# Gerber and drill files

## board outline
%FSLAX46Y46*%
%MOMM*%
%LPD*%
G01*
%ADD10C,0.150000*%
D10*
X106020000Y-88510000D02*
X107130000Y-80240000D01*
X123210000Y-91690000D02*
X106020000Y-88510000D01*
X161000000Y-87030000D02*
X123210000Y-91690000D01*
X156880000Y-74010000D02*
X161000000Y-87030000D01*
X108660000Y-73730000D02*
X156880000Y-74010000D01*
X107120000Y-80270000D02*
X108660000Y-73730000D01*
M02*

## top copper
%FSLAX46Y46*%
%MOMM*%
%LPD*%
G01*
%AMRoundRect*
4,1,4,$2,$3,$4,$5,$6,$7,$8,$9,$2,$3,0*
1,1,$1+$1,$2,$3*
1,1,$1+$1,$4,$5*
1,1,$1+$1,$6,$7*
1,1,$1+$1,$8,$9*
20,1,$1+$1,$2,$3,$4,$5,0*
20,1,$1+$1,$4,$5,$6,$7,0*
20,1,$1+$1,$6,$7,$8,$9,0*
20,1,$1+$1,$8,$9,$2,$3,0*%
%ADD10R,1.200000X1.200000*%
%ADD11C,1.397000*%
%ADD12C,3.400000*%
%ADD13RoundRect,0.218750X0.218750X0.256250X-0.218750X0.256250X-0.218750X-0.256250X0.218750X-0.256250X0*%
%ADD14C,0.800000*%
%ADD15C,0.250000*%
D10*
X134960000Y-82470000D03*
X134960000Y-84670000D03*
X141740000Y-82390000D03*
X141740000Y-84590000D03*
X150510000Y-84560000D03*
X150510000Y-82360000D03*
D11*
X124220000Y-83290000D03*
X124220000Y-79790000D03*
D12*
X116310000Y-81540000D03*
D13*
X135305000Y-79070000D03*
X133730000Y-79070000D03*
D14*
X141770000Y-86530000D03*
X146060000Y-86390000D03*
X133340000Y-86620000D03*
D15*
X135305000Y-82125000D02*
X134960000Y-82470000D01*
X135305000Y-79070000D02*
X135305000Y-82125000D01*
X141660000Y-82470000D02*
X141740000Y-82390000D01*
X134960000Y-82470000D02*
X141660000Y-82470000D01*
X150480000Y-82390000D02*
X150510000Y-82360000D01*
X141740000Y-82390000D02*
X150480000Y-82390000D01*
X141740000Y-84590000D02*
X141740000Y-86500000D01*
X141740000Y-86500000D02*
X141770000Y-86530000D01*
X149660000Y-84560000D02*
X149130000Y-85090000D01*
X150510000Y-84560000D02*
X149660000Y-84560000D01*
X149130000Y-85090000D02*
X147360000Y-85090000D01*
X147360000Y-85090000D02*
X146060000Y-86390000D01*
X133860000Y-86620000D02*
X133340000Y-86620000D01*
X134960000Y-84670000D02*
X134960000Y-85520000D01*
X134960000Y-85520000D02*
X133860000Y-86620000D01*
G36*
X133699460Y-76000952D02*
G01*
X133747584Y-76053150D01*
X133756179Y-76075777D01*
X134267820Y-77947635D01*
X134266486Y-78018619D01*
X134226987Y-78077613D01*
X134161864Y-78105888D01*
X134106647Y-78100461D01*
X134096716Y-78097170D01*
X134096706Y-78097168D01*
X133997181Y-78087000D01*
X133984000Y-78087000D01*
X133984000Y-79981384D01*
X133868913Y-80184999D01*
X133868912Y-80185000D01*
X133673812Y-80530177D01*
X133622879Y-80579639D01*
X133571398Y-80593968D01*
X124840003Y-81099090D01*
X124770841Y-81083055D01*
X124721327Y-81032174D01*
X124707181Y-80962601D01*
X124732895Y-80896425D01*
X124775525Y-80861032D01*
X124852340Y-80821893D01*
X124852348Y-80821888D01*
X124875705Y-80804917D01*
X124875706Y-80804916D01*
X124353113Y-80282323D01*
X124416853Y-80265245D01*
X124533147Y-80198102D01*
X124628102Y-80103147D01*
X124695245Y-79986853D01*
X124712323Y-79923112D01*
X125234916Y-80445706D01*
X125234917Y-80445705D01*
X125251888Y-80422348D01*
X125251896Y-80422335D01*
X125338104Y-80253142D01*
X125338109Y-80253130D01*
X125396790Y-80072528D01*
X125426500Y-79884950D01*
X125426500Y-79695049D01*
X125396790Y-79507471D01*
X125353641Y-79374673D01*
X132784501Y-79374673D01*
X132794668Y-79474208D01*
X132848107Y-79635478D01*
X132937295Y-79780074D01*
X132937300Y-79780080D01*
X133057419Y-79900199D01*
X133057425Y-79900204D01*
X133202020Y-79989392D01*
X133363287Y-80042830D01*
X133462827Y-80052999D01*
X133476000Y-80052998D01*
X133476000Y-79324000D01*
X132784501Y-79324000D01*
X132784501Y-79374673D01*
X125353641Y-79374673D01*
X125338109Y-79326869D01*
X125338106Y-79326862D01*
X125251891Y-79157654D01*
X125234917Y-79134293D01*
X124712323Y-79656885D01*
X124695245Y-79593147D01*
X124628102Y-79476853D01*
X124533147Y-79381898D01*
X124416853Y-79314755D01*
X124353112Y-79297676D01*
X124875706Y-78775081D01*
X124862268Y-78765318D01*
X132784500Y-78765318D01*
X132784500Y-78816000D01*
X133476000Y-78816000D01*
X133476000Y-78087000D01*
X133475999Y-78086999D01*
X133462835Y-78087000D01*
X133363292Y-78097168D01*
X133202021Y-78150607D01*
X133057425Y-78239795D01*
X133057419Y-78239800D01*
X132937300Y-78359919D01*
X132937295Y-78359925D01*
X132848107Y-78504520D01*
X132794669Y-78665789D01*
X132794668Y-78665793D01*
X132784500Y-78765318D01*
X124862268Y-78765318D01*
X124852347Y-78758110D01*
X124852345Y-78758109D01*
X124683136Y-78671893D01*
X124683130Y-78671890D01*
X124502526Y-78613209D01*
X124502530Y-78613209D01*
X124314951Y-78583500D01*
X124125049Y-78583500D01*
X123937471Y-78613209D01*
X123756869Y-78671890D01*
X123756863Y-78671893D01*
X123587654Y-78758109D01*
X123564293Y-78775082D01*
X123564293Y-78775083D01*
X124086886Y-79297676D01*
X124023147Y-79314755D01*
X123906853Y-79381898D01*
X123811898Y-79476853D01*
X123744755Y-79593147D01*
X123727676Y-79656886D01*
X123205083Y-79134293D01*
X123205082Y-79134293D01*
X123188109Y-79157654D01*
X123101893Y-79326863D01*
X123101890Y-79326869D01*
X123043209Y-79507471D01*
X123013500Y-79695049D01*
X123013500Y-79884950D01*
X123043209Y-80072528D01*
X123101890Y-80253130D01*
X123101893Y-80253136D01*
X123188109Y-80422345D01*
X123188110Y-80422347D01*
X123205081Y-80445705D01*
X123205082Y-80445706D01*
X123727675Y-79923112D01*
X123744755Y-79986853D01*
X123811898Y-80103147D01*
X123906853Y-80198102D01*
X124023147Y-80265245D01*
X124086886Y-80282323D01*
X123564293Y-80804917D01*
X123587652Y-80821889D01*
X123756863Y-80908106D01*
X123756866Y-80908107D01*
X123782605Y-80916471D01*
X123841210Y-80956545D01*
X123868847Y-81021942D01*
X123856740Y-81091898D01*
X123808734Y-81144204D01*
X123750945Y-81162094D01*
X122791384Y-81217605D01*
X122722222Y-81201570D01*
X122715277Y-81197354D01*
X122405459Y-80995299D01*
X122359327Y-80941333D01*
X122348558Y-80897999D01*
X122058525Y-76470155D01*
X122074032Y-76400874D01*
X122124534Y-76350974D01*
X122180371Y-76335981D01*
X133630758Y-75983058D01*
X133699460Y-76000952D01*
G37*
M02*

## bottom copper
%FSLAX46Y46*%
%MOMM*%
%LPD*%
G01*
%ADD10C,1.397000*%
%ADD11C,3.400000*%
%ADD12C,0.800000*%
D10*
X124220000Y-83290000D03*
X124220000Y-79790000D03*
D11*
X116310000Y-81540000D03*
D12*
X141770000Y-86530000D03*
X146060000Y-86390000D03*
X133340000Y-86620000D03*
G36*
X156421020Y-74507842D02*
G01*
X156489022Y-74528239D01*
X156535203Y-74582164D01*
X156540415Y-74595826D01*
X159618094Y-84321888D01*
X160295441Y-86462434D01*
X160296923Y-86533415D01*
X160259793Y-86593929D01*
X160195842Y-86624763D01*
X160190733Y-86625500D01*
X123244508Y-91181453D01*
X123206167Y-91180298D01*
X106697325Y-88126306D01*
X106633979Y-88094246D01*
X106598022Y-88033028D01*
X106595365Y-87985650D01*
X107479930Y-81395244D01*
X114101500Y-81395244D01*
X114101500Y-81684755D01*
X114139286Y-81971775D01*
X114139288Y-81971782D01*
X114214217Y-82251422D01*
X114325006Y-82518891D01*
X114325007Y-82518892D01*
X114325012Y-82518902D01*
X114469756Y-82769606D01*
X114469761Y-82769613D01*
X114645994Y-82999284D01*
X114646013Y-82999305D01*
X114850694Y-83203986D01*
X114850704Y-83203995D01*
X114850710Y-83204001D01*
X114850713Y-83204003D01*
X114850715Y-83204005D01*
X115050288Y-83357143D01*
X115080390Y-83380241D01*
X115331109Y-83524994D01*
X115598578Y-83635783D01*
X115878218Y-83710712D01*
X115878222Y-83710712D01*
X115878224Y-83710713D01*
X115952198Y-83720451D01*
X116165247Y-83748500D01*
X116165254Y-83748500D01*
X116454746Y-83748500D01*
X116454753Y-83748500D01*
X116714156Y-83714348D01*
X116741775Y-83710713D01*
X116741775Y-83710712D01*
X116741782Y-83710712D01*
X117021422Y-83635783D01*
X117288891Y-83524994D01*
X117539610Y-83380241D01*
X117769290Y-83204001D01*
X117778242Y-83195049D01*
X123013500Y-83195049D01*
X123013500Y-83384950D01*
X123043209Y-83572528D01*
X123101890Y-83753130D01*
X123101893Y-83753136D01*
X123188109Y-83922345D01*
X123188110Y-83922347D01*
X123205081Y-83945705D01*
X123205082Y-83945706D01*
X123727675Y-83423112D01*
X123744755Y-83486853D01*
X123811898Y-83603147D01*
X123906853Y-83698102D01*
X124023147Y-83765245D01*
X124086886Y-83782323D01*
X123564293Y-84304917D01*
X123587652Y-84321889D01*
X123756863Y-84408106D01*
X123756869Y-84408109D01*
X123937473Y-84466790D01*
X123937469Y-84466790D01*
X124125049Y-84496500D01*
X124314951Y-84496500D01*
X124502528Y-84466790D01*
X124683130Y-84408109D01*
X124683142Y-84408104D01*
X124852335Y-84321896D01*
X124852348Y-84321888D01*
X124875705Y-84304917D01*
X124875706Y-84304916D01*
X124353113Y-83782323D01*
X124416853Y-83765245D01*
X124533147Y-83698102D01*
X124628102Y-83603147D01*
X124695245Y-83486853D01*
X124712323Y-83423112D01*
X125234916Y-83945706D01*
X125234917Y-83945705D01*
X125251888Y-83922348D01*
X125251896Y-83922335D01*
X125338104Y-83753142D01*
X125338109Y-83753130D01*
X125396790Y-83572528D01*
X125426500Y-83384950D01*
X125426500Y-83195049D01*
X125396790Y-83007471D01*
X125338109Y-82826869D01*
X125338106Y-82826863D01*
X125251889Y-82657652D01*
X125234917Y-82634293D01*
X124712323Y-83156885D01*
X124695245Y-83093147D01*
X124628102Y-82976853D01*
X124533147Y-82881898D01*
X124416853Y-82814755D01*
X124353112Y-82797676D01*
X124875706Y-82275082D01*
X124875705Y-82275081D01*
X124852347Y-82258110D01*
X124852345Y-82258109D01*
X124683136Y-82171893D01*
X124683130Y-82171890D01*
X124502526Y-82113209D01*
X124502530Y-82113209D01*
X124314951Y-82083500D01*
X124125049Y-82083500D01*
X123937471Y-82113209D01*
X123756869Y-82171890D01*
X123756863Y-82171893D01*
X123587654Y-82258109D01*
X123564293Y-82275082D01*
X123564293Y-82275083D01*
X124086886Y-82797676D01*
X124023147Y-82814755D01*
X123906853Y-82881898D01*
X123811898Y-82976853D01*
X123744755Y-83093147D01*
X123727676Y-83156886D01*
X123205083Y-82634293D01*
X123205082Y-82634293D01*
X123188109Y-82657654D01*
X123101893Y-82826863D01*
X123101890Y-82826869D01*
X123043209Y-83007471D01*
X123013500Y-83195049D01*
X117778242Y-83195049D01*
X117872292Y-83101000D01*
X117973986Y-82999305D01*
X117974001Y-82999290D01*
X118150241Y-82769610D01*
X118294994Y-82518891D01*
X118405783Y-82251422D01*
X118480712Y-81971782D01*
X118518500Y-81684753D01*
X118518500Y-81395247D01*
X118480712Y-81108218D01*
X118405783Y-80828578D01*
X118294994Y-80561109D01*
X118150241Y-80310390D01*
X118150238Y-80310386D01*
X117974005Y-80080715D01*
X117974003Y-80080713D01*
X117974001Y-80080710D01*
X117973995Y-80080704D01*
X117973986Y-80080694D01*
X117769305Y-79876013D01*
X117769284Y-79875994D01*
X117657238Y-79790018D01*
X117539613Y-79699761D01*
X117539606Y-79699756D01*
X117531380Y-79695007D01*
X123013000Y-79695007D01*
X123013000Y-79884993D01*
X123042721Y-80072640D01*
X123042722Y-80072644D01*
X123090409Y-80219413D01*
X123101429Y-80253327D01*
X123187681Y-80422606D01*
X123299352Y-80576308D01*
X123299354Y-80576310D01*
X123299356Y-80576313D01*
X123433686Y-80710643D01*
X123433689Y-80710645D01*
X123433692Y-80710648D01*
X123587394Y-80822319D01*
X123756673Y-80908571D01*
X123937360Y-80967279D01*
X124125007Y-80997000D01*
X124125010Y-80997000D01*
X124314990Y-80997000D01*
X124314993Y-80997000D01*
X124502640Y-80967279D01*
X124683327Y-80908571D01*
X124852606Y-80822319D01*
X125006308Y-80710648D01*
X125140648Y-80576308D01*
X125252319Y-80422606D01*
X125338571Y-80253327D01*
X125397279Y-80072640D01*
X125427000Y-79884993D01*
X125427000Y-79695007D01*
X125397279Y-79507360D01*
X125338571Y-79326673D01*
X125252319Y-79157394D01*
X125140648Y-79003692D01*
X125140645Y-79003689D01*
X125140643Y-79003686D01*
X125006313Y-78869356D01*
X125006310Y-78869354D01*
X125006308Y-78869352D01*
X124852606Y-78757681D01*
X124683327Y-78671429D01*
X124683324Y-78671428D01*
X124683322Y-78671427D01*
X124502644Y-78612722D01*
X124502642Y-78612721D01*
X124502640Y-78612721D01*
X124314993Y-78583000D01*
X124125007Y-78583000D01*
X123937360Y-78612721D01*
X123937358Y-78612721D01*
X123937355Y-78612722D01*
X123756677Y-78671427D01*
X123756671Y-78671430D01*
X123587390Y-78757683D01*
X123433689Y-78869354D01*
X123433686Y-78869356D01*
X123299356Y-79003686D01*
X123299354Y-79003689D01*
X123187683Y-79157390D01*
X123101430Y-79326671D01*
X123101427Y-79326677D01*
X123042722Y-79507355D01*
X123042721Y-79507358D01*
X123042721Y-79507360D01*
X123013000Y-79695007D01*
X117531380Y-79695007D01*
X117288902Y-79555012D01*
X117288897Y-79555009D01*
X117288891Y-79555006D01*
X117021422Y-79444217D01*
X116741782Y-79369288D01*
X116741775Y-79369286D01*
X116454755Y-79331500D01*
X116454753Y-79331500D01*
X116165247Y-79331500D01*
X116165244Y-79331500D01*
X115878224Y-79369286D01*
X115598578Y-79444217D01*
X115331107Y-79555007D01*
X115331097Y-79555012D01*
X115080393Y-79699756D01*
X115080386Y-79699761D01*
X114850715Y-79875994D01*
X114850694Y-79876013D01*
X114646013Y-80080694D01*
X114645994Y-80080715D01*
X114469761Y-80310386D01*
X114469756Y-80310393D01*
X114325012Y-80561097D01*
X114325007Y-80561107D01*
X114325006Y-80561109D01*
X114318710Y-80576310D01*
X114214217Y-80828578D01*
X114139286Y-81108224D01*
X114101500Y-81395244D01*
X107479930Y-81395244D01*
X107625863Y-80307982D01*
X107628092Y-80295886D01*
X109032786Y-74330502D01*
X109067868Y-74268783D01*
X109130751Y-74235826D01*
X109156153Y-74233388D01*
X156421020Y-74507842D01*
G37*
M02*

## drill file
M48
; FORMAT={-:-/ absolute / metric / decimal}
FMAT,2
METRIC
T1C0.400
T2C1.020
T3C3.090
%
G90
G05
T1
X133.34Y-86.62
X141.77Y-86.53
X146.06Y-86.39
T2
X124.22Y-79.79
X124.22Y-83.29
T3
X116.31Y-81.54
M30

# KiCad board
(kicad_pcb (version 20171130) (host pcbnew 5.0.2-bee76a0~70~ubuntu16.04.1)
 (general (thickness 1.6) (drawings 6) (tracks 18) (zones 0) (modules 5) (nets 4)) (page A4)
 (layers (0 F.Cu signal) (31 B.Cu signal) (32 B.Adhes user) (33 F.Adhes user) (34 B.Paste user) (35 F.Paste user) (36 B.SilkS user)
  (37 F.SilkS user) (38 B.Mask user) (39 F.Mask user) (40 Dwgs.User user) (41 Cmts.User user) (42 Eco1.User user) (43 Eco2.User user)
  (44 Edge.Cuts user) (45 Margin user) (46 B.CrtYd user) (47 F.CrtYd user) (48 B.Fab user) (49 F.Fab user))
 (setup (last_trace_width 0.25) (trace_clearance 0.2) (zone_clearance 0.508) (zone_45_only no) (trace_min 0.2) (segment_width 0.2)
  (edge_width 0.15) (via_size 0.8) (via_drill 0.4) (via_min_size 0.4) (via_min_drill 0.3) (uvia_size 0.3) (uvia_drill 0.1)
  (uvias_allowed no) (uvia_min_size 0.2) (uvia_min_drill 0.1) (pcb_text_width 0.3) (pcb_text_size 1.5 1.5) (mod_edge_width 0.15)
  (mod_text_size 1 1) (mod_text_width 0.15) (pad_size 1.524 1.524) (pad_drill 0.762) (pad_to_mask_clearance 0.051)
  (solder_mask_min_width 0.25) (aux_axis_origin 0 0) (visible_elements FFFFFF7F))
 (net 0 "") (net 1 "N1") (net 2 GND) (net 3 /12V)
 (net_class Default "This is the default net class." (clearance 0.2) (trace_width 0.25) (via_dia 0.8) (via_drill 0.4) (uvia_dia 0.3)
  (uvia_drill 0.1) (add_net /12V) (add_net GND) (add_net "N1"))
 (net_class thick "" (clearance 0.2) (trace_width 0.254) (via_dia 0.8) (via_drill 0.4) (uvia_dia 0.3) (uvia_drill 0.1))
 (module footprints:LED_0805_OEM (layer F.Cu) (at 134.96 83.57 90)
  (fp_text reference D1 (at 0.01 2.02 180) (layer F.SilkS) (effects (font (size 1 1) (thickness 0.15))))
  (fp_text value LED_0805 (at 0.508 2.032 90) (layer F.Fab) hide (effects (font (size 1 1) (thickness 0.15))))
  (pad 2 smd rect (at 1.1 0 270) (size 1.2 1.2) (layers F.Cu F.Paste F.Mask) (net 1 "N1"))
  (pad 1 smd rect (at -1.1 0 270) (size 1.2 1.2) (layers F.Cu F.Paste F.Mask) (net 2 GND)))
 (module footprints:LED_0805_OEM (layer F.Cu) (at 141.74 83.49 90)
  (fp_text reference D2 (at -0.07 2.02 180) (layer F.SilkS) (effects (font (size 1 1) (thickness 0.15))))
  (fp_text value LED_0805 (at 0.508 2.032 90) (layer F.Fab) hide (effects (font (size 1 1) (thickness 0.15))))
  (pad 2 smd rect (at 1.1 0 270) (size 1.2 1.2) (layers F.Cu F.Paste F.Mask) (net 1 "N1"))
  (pad 1 smd rect (at -1.1 0 270) (size 1.2 1.2) (layers F.Cu F.Paste F.Mask) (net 2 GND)))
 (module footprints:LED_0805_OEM (layer F.Cu) (at 150.51 83.46 90)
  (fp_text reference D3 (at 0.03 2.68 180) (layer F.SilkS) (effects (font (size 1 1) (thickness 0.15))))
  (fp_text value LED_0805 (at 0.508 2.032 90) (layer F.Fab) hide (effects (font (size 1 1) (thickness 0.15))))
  (pad 1 smd rect (at -1.1 0 270) (size 1.2 1.2) (layers F.Cu F.Paste F.Mask) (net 2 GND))
  (pad 2 smd rect (at 1.1 0 270) (size 1.2 1.2) (layers F.Cu F.Paste F.Mask) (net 1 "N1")))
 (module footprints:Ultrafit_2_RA (layer F.Cu) (at 124.22 83.29 180)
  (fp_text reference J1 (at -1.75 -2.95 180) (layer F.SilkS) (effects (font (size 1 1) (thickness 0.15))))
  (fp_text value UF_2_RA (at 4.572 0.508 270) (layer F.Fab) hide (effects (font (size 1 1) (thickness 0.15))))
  (pad 2 thru_hole circle (at 0 0 180) (size 1.397 1.397) (drill 1.02) (layers *.Cu *.Mask) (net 2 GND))
  (pad 1 thru_hole circle (at 0 3.5 180) (size 1.397 1.397) (drill 1.02) (layers *.Cu *.Mask) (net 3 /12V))
  (pad "" thru_hole circle (at 7.91 1.75 180) (size 3.4 3.4) (drill 3.09) (layers *.Cu *.Mask)))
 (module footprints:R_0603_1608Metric (layer F.Cu) (at 134.5175 79.07 180)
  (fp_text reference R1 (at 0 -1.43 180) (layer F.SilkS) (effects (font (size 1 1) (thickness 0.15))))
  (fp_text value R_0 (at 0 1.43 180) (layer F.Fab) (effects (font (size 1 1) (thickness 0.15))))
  (pad 1 smd roundrect (at -0.7875 0 180) (size 0.875 0.95) (layers F.Cu F.Paste F.Mask) (roundrect_rratio 0.25) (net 1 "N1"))
  (pad 2 smd roundrect (at 0.7875 0 180) (size 0.875 0.95) (layers F.Cu F.Paste F.Mask) (roundrect_rratio 0.25) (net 3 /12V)))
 (gr_line (start 106.02 88.51) (end 107.13 80.24) (layer Edge.Cuts) (width 0.15))
 (gr_line (start 123.21 91.69) (end 106.02 88.51) (layer Edge.Cuts) (width 0.15))
 (gr_line (start 161 87.03) (end 123.21 91.69) (layer Edge.Cuts) (width 0.15))
 (gr_line (start 156.88 74.01) (end 161 87.03) (layer Edge.Cuts) (width 0.15))
 (gr_line (start 108.66 73.73) (end 156.88 74.01) (layer Edge.Cuts) (width 0.15))
 (gr_line (start 107.12 80.27) (end 108.66 73.73) (layer Edge.Cuts) (width 0.15))
 (segment (start 135.305 82.125) (end 134.96 82.47) (width 0.25) (layer F.Cu) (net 1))
 (segment (start 135.305 79.07) (end 135.305 82.125) (width 0.25) (layer F.Cu) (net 1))
 (segment (start 141.66 82.47) (end 141.74 82.39) (width 0.25) (layer F.Cu) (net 1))
 (segment (start 134.96 82.47) (end 141.66 82.47) (width 0.25) (layer F.Cu) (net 1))
 (segment (start 150.48 82.39) (end 150.51 82.36) (width 0.25) (layer F.Cu) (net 1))
 (segment (start 141.74 82.39) (end 150.48 82.39) (width 0.25) (layer F.Cu) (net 1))
 (via (at 141.77 86.53) (size 0.8) (drill 0.4) (layers F.Cu B.Cu) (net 2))
 (segment (start 141.74 84.59) (end 141.74 86.5) (width 0.25) (layer F.Cu) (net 2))
 (segment (start 141.74 86.5) (end 141.77 86.53) (width 0.25) (layer F.Cu) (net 2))
 (segment (start 149.66 84.56) (end 149.13 85.09) (width 0.25) (layer F.Cu) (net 2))
 (segment (start 150.51 84.56) (end 149.66 84.56) (width 0.25) (layer F.Cu) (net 2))
 (segment (start 149.13 85.09) (end 147.36 85.09) (width 0.25) (layer F.Cu) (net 2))
 (via (at 146.06 86.39) (size 0.8) (drill 0.4) (layers F.Cu B.Cu) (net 2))
 (segment (start 147.36 85.09) (end 146.06 86.39) (width 0.25) (layer F.Cu) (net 2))
 (via (at 133.34 86.62) (size 0.8) (drill 0.4) (layers F.Cu B.Cu) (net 2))
 (segment (start 133.86 86.62) (end 133.34 86.62) (width 0.25) (layer F.Cu) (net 2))
 (segment (start 134.96 84.67) (end 134.96 85.52) (width 0.25) (layer F.Cu) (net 2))
 (segment (start 134.96 85.52) (end 133.86 86.62) (width 0.25) (layer F.Cu) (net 2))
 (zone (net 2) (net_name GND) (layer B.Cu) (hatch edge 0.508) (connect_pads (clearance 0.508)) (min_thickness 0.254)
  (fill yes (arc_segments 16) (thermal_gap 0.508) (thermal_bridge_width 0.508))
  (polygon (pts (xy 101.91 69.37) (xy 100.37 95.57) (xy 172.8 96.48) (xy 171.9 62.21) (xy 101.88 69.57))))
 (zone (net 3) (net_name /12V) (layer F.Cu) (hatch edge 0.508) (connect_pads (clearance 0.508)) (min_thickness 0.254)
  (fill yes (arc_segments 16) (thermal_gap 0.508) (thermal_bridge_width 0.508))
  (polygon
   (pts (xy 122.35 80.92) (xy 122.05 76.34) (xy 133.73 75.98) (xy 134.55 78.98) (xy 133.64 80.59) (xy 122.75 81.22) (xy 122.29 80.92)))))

